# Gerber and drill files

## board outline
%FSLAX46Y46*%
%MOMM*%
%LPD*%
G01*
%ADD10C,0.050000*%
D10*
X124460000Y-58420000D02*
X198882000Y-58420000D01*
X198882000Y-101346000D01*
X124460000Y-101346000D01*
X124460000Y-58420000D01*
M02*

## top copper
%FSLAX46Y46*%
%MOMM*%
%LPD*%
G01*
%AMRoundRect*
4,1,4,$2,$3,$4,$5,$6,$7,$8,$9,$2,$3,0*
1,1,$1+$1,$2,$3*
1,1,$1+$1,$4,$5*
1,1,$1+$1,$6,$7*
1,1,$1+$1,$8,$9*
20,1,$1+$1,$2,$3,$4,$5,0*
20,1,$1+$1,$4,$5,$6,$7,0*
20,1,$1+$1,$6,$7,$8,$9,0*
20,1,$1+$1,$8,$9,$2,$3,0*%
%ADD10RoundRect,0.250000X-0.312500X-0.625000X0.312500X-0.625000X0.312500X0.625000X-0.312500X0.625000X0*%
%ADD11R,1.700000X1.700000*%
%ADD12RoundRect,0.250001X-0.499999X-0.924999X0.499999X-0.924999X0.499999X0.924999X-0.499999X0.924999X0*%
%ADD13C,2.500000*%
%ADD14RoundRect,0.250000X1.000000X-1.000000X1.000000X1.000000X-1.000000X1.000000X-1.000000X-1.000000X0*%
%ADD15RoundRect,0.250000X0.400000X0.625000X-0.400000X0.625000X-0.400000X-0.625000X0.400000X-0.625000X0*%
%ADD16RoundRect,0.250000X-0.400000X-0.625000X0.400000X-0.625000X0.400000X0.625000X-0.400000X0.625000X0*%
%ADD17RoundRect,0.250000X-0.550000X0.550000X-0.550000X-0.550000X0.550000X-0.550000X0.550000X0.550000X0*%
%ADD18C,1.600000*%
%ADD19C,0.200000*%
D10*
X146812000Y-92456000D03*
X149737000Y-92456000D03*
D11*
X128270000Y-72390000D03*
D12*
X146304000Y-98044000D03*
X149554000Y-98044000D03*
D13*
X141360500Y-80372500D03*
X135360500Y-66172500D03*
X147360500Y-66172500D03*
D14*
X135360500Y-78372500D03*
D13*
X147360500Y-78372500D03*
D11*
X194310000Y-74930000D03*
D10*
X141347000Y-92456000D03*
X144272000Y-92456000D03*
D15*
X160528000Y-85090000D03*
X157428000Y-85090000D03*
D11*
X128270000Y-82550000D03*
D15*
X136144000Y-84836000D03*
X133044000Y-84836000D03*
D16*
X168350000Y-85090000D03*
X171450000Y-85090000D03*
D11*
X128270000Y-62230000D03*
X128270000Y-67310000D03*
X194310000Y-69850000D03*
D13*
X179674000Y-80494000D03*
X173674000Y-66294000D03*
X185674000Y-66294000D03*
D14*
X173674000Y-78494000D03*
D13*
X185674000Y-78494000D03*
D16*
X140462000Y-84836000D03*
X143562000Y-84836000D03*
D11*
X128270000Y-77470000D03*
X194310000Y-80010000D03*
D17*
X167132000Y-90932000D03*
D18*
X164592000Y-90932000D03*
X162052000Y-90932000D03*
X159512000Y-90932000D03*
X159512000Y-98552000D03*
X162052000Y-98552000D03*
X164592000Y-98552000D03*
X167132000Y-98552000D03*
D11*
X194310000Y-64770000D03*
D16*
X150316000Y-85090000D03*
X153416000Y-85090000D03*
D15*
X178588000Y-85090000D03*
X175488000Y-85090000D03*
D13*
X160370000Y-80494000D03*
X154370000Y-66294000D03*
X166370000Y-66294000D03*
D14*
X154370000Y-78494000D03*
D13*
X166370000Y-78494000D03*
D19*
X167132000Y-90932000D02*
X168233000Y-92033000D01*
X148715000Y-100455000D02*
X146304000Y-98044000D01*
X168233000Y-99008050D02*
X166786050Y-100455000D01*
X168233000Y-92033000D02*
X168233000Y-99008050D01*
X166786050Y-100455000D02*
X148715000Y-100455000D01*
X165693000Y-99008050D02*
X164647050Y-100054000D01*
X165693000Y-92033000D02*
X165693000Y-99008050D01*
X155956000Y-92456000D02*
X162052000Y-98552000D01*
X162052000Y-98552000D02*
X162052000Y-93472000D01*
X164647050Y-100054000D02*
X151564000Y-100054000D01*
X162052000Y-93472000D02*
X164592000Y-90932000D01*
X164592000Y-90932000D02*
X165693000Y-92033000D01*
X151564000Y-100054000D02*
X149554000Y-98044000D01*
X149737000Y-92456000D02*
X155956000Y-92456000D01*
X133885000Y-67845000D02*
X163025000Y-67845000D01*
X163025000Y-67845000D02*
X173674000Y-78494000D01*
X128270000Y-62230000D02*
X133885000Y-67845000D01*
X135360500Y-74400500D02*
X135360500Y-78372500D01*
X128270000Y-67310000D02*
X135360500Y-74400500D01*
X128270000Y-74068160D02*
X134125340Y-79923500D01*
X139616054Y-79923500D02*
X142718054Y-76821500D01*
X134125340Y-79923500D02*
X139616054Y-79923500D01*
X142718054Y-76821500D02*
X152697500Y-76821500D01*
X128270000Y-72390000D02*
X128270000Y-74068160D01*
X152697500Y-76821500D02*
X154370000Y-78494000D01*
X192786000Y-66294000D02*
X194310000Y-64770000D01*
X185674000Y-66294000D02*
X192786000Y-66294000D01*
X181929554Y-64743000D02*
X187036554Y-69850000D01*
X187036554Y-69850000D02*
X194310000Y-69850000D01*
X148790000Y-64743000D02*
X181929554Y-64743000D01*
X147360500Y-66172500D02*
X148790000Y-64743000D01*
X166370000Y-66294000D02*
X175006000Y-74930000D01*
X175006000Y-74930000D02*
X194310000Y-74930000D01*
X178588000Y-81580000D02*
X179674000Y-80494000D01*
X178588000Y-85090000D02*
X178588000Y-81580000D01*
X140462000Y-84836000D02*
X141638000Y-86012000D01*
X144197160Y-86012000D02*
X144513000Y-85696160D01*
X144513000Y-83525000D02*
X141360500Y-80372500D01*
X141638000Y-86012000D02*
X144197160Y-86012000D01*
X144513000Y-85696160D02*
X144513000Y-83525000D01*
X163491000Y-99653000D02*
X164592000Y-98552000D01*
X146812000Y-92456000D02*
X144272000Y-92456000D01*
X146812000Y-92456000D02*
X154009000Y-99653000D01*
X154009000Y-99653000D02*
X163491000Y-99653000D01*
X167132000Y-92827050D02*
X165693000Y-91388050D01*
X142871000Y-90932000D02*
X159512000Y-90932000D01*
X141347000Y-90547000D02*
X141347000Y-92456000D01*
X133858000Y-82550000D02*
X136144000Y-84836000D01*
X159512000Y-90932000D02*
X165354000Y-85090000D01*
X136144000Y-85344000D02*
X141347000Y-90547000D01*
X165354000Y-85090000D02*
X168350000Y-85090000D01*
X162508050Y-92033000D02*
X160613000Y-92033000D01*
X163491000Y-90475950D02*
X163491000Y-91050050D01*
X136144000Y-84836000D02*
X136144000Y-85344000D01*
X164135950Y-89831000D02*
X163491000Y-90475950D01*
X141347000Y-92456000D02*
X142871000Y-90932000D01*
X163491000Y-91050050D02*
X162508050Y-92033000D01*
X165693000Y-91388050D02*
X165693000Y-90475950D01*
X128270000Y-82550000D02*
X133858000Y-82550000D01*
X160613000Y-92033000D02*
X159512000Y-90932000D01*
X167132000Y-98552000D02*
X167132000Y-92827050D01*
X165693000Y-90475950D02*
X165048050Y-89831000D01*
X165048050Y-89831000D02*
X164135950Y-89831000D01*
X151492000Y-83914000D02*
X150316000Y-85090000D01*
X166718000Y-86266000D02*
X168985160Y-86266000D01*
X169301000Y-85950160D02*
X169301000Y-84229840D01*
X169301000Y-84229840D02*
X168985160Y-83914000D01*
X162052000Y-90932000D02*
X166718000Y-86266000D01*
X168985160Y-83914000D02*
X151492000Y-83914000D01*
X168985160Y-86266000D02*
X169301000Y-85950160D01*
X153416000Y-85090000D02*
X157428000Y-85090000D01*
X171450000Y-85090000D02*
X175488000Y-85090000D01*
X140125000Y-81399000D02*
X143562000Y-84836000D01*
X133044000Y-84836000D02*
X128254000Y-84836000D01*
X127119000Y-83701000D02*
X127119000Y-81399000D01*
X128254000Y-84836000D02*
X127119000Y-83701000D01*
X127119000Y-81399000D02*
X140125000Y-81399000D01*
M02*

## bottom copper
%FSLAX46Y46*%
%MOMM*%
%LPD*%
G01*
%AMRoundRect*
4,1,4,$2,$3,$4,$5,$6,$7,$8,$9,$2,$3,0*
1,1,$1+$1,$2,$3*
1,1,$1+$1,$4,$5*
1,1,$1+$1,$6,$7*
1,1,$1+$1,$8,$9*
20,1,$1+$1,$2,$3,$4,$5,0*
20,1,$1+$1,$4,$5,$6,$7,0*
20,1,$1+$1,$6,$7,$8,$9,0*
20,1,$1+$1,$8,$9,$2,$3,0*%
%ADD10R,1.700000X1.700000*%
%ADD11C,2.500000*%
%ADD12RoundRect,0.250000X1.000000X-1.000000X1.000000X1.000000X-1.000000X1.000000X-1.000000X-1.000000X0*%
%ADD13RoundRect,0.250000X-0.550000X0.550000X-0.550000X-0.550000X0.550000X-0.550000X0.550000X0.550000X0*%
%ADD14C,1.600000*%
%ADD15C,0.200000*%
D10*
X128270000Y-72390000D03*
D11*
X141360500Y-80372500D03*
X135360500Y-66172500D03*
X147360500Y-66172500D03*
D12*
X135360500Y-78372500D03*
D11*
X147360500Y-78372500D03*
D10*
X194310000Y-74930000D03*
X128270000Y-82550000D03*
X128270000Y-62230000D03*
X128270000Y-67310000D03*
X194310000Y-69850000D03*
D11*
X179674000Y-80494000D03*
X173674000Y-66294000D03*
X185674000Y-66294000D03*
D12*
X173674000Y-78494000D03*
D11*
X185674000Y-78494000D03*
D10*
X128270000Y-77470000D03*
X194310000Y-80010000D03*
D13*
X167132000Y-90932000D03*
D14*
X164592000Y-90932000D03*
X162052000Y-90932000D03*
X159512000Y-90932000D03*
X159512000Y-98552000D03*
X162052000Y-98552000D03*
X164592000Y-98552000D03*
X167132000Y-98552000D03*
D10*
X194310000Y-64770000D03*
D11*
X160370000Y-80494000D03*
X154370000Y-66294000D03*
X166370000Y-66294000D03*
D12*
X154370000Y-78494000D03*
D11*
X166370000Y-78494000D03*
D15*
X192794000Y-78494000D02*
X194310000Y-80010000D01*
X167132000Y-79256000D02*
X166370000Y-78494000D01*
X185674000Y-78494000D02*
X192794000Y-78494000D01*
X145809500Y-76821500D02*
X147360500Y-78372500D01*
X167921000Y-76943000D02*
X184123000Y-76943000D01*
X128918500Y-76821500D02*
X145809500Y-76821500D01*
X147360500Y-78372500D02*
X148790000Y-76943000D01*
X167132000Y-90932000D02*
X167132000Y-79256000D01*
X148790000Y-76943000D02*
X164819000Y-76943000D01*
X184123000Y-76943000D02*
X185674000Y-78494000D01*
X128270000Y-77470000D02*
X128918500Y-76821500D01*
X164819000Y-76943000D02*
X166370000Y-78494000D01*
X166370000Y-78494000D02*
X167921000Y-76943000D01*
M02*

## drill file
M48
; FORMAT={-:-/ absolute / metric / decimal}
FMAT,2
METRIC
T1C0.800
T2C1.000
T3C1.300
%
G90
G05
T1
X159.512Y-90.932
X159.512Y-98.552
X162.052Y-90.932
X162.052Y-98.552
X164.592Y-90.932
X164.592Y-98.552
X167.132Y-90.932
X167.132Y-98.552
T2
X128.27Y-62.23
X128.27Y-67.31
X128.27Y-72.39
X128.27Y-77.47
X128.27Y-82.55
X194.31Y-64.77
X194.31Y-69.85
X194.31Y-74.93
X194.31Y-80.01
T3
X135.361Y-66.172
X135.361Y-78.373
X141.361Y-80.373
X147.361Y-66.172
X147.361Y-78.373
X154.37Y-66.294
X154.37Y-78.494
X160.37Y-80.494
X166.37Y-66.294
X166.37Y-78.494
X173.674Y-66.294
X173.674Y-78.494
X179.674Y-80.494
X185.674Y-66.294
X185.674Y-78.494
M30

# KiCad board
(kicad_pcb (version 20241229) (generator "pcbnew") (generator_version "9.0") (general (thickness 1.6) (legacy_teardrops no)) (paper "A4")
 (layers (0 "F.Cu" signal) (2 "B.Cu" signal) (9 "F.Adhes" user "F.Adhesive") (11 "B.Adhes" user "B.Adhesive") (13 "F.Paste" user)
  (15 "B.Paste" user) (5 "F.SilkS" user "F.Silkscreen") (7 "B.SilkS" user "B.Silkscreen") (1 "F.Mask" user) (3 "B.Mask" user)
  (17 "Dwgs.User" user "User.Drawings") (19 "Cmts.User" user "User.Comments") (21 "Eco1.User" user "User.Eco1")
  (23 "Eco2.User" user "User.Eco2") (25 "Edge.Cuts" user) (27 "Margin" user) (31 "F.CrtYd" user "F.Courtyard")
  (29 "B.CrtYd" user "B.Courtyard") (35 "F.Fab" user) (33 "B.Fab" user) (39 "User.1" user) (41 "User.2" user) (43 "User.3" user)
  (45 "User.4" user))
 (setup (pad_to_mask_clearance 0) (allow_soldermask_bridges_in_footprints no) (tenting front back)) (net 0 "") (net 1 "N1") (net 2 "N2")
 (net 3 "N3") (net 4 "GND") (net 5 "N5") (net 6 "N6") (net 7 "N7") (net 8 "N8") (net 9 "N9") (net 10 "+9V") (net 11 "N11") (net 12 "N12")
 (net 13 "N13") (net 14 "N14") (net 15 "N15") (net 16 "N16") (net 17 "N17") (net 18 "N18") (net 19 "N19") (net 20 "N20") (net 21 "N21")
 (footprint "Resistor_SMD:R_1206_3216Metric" (layer "F.Cu") (at 148.2745 92.456)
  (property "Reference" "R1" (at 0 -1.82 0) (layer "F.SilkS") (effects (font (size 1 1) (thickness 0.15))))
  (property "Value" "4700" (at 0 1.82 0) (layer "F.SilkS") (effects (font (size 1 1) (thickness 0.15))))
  (pad "1" smd roundrect (at -1.4625 0) (size 1.125 1.75) (layers "F.Cu" "F.Mask" "F.Paste") (roundrect_rratio 0.222222) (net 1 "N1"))
  (pad "2" smd roundrect (at 1.4625 0) (size 1.125 1.75) (layers "F.Cu" "F.Mask" "F.Paste") (roundrect_rratio 0.222222) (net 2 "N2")))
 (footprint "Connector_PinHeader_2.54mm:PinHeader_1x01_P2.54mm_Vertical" (layer "F.Cu") (at 128.27 72.39 -90)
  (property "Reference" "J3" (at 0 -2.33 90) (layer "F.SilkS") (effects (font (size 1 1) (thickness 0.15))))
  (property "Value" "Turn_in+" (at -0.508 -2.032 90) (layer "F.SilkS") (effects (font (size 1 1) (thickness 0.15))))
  (pad "1" thru_hole rect (at 0 0 270) (size 1.7 1.7) (drill 1) (layers "*.Cu" "*.Mask") (remove_unused_layers no) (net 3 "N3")))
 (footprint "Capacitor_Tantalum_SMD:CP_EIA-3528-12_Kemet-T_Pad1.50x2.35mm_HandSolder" (layer "F.Cu") (at 147.929 98.044)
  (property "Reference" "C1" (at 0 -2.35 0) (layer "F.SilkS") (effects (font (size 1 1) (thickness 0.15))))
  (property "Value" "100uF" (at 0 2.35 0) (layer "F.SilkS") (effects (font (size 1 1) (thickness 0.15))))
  (pad "1" smd roundrect (at -1.625 0) (size 1.5 2.35) (layers "F.Cu" "F.Mask" "F.Paste") (roundrect_rratio 0.166667) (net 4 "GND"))
  (pad "2" smd roundrect (at 1.625 0) (size 1.5 2.35) (layers "F.Cu" "F.Mask" "F.Paste") (roundrect_rratio 0.166667) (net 2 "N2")))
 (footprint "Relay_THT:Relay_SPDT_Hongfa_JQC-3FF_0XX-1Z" (layer "F.Cu") (at 135.3605 78.3725 90)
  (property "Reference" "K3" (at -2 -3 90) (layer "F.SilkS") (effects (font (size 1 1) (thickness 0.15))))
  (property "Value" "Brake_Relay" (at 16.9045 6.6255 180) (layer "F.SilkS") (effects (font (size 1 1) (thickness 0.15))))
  (pad "11" thru_hole circle (at -2 6 90) (size 2.5 2.5) (drill 1.3) (layers "*.Cu" "*.Mask") (remove_unused_layers no) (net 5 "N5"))
  (pad "12" thru_hole circle (at 12.2 0 90) (size 2.5 2.5) (drill 1.3) (layers "*.Cu" "*.Mask") (remove_unused_layers no) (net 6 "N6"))
  (pad "14" thru_hole circle (at 12.2 12 90) (size 2.5 2.5) (drill 1.3) (layers "*.Cu" "*.Mask") (remove_unused_layers no) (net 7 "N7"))
  (pad "A1" thru_hole roundrect (at 0 0 90) (size 2.5 2.5) (drill 1.3) (layers "*.Cu" "*.Mask") (remove_unused_layers no)
   (roundrect_rratio 0.1) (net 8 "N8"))
  (pad "A2" thru_hole circle (at 0 12 90) (size 2.5 2.5) (drill 1.3) (layers "*.Cu" "*.Mask") (remove_unused_layers no) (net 4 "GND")))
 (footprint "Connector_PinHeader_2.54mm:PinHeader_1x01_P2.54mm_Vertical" (layer "F.Cu") (at 194.31 74.93 -90)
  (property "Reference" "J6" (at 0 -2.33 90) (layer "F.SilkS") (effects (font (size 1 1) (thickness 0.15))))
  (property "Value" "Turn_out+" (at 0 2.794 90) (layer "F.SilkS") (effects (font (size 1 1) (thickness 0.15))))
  (pad "1" thru_hole rect (at 0 0 270) (size 1.7 1.7) (drill 1) (layers "*.Cu" "*.Mask") (remove_unused_layers no) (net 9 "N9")))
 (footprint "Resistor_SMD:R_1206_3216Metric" (layer "F.Cu") (at 142.8095 92.456)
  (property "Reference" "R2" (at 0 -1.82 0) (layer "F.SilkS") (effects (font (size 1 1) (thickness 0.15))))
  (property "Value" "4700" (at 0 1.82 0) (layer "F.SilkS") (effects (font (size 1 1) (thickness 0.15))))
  (pad "1" smd roundrect (at -1.4625 0) (size 1.125 1.75) (layers "F.Cu" "F.Mask" "F.Paste") (roundrect_rratio 0.222222) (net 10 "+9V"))
  (pad "2" smd roundrect (at 1.4625 0) (size 1.125 1.75) (layers "F.Cu" "F.Mask" "F.Paste") (roundrect_rratio 0.222222) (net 1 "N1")))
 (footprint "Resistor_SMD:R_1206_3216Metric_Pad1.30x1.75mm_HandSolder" (layer "F.Cu") (at 158.978 85.09 180)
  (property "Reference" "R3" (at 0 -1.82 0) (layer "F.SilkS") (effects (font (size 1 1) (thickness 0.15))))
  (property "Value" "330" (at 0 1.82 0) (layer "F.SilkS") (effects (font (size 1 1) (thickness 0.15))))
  (pad "1" smd roundrect (at -1.55 0 180) (size 1.3 1.75) (layers "F.Cu" "F.Mask" "F.Paste") (roundrect_rratio 0.192308) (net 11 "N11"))
  (pad "2" smd roundrect (at 1.55 0 180) (size 1.3 1.75) (layers "F.Cu" "F.Mask" "F.Paste") (roundrect_rratio 0.192308) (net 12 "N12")))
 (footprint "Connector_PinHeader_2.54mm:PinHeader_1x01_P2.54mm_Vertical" (layer "F.Cu") (at 128.27 82.55 -90)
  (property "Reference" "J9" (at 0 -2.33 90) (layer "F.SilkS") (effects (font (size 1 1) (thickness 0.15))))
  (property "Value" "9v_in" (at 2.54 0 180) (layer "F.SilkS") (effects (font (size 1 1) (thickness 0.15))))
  (pad "1" thru_hole rect (at 0 0 270) (size 1.7 1.7) (drill 1) (layers "*.Cu" "*.Mask") (remove_unused_layers no) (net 10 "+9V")))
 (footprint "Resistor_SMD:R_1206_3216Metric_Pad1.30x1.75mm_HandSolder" (layer "F.Cu") (at 134.594 84.836 180)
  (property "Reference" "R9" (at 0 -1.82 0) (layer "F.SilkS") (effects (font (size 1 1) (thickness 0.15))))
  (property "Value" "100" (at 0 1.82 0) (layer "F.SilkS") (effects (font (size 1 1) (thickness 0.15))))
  (pad "1" smd roundrect (at -1.55 0 180) (size 1.3 1.75) (layers "F.Cu" "F.Mask" "F.Paste") (roundrect_rratio 0.192308) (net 10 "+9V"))
  (pad "2" smd roundrect (at 1.55 0 180) (size 1.3 1.75) (layers "F.Cu" "F.Mask" "F.Paste") (roundrect_rratio 0.192308) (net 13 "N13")))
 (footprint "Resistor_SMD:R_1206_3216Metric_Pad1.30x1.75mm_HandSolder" (layer "F.Cu") (at 169.9 85.09)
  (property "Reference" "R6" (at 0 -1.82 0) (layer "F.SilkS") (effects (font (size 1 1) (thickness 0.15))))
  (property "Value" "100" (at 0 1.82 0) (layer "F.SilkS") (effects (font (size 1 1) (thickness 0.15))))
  (pad "1" smd roundrect (at -1.55 0) (size 1.3 1.75) (layers "F.Cu" "F.Mask" "F.Paste") (roundrect_rratio 0.192308) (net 10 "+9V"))
  (pad "2" smd roundrect (at 1.55 0) (size 1.3 1.75) (layers "F.Cu" "F.Mask" "F.Paste") (roundrect_rratio 0.192308) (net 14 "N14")))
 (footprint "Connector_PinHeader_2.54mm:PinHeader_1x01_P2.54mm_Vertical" (layer "F.Cu") (at 128.27 62.23 -90)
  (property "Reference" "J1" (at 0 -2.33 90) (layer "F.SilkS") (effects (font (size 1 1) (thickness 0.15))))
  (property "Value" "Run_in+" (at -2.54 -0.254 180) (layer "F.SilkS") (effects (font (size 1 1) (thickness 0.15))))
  (pad "1" thru_hole rect (at 0 0 270) (size 1.7 1.7) (drill 1) (layers "*.Cu" "*.Mask") (remove_unused_layers no) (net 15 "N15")))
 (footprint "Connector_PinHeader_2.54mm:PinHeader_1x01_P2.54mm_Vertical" (layer "F.Cu") (at 128.27 67.31 -90)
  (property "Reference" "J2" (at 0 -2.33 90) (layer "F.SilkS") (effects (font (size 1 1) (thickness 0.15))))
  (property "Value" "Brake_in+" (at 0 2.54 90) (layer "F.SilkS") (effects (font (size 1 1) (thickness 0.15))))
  (pad "1" thru_hole rect (at 0 0 270) (size 1.7 1.7) (drill 1) (layers "*.Cu" "*.Mask") (remove_unused_layers no) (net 8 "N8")))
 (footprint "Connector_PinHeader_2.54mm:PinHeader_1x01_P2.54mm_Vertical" (layer "F.Cu") (at 194.31 69.85 -90)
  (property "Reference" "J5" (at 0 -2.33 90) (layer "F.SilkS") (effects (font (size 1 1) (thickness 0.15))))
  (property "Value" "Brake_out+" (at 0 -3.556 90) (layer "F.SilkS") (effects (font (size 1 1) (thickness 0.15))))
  (pad "1" thru_hole rect (at 0 0 270) (size 1.7 1.7) (drill 1) (layers "*.Cu" "*.Mask") (remove_unused_layers no) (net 7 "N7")))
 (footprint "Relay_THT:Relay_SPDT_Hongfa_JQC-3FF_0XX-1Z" (layer "F.Cu") (at 173.674 78.494 90)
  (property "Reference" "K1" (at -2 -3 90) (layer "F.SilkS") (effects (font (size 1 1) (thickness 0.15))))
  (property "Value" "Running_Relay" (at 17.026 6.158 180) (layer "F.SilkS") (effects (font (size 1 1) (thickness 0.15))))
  (pad "11" thru_hole circle (at -2 6 90) (size 2.5 2.5) (drill 1.3) (layers "*.Cu" "*.Mask") (remove_unused_layers no) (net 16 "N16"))
  (pad "12" thru_hole circle (at 12.2 0 90) (size 2.5 2.5) (drill 1.3) (layers "*.Cu" "*.Mask") (remove_unused_layers no) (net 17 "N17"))
  (pad "14" thru_hole circle (at 12.2 12 90) (size 2.5 2.5) (drill 1.3) (layers "*.Cu" "*.Mask") (remove_unused_layers no) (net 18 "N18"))
  (pad "A1" thru_hole roundrect (at 0 0 90) (size 2.5 2.5) (drill 1.3) (layers "*.Cu" "*.Mask") (remove_unused_layers no)
   (roundrect_rratio 0.1) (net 15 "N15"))
  (pad "A2" thru_hole circle (at 0 12 90) (size 2.5 2.5) (drill 1.3) (layers "*.Cu" "*.Mask") (remove_unused_layers no) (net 4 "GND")))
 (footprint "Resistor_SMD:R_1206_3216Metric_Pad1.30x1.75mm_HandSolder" (layer "F.Cu") (at 142.012 84.836)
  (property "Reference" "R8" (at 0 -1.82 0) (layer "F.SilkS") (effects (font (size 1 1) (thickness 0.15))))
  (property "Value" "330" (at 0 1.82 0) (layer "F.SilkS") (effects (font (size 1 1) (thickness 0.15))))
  (pad "1" smd roundrect (at -1.55 0) (size 1.3 1.75) (layers "F.Cu" "F.Mask" "F.Paste") (roundrect_rratio 0.192308) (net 5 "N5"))
  (pad "2" smd roundrect (at 1.55 0) (size 1.3 1.75) (layers "F.Cu" "F.Mask" "F.Paste") (roundrect_rratio 0.192308) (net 13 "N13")))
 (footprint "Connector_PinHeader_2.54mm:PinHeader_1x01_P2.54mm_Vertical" (layer "F.Cu") (at 128.27 77.47 -90)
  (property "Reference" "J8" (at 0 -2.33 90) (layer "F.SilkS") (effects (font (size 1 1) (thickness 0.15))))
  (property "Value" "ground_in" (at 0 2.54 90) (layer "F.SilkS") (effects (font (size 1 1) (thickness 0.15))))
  (pad "1" thru_hole rect (at 0 0 270) (size 1.7 1.7) (drill 1) (layers "*.Cu" "*.Mask") (remove_unused_layers no) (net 4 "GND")))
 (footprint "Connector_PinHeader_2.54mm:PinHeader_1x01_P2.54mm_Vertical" (layer "F.Cu") (at 194.31 80.01 -90)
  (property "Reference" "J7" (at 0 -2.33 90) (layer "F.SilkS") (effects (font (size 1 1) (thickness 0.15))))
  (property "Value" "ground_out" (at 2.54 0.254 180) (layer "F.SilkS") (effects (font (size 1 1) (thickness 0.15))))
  (pad "1" thru_hole rect (at 0 0 270) (size 1.7 1.7) (drill 1) (layers "*.Cu" "*.Mask") (remove_unused_layers no) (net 4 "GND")))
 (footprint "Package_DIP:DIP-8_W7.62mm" (layer "F.Cu") (at 167.132 90.932 -90)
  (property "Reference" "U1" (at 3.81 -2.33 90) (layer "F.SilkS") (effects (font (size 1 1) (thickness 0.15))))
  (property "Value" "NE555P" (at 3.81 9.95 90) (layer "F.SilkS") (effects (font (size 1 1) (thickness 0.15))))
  (pad "1" thru_hole roundrect (at 0 0 270) (size 1.6 1.6) (drill 0.8) (layers "*.Cu" "*.Mask") (remove_unused_layers no)
   (roundrect_rratio 0.15625) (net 4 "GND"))
  (pad "2" thru_hole circle (at 0 2.54 270) (size 1.6 1.6) (drill 0.8) (layers "*.Cu" "*.Mask") (remove_unused_layers no) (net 2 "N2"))
  (pad "3" thru_hole circle (at 0 5.08 270) (size 1.6 1.6) (drill 0.8) (layers "*.Cu" "*.Mask") (remove_unused_layers no) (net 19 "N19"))
  (pad "4" thru_hole circle (at 0 7.62 270) (size 1.6 1.6) (drill 0.8) (layers "*.Cu" "*.Mask") (remove_unused_layers no) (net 10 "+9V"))
  (pad "5" thru_hole circle (at 7.62 7.62 270) (size 1.6 1.6) (drill 0.8) (layers "*.Cu" "*.Mask") (remove_unused_layers no) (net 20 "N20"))
  (pad "6" thru_hole circle (at 7.62 5.08 270) (size 1.6 1.6) (drill 0.8) (layers "*.Cu" "*.Mask") (remove_unused_layers no) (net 2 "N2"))
  (pad "7" thru_hole circle (at 7.62 2.54 270) (size 1.6 1.6) (drill 0.8) (layers "*.Cu" "*.Mask") (remove_unused_layers no) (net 1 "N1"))
  (pad "8" thru_hole circle (at 7.62 0 270) (size 1.6 1.6) (drill 0.8) (layers "*.Cu" "*.Mask") (remove_unused_layers no) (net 10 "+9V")))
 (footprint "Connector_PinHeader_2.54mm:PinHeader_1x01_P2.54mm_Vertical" (layer "F.Cu") (at 194.31 64.77 -90)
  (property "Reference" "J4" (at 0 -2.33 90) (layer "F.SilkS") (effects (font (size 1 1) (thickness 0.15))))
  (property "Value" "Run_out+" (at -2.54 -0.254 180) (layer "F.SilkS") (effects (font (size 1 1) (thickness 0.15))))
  (pad "1" thru_hole rect (at 0 0 270) (size 1.7 1.7) (drill 1) (layers "*.Cu" "*.Mask") (remove_unused_layers no) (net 18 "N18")))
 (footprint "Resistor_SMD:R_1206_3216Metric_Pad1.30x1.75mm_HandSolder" (layer "F.Cu") (at 151.866 85.09)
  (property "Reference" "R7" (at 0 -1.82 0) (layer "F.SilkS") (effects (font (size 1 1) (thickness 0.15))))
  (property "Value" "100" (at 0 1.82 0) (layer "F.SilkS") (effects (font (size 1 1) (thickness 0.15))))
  (pad "1" smd roundrect (at -1.55 0) (size 1.3 1.75) (layers "F.Cu" "F.Mask" "F.Paste") (roundrect_rratio 0.192308) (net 19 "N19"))
  (pad "2" smd roundrect (at 1.55 0) (size 1.3 1.75) (layers "F.Cu" "F.Mask" "F.Paste") (roundrect_rratio 0.192308) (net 12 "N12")))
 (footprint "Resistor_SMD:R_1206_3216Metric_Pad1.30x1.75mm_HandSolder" (layer "F.Cu") (at 177.038 85.09 180)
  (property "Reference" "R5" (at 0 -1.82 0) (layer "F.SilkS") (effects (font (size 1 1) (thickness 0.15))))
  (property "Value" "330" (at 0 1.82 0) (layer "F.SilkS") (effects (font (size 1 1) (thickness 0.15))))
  (pad "1" smd roundrect (at -1.55 0 180) (size 1.3 1.75) (layers "F.Cu" "F.Mask" "F.Paste") (roundrect_rratio 0.192308) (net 16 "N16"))
  (pad "2" smd roundrect (at 1.55 0 180) (size 1.3 1.75) (layers "F.Cu" "F.Mask" "F.Paste") (roundrect_rratio 0.192308) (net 14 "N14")))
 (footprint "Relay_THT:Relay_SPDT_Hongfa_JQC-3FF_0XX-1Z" (layer "F.Cu") (at 154.37 78.494 90)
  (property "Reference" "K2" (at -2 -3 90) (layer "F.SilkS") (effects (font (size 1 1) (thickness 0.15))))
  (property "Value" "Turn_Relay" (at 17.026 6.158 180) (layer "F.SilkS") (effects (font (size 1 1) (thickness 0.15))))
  (pad "11" thru_hole circle (at -2 6 90) (size 2.5 2.5) (drill 1.3) (layers "*.Cu" "*.Mask") (remove_unused_layers no) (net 11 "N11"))
  (pad "12" thru_hole circle (at 12.2 0 90) (size 2.5 2.5) (drill 1.3) (layers "*.Cu" "*.Mask") (remove_unused_layers no) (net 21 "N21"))
  (pad "14" thru_hole circle (at 12.2 12 90) (size 2.5 2.5) (drill 1.3) (layers "*.Cu" "*.Mask") (remove_unused_layers no) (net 9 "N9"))
  (pad "A1" thru_hole roundrect (at 0 0 90) (size 2.5 2.5) (drill 1.3) (layers "*.Cu" "*.Mask") (remove_unused_layers no)
   (roundrect_rratio 0.1) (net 3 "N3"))
  (pad "A2" thru_hole circle (at 0 12 90) (size 2.5 2.5) (drill 1.3) (layers "*.Cu" "*.Mask") (remove_unused_layers no) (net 4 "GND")))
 (gr_rect (start 124.46 58.42) (end 198.882 101.346) (stroke (width 0.05) (type default)) (fill no) (layer "Edge.Cuts"))
 (segment (start 167.132 90.932) (end 168.233 92.033) (width 0.2) (layer "F.Cu") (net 4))
 (segment (start 148.715 100.455) (end 146.304 98.044) (width 0.2) (layer "F.Cu") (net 4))
 (segment (start 168.233 99.00805) (end 166.78605 100.455) (width 0.2) (layer "F.Cu") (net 4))
 (segment (start 168.233 92.033) (end 168.233 99.00805) (width 0.2) (layer "F.Cu") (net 4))
 (segment (start 166.78605 100.455) (end 148.715 100.455) (width 0.2) (layer "F.Cu") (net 4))
 (segment (start 192.794 78.494) (end 194.31 80.01) (width 0.2) (layer "B.Cu") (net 4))
 (segment (start 167.132 79.256) (end 166.37 78.494) (width 0.2) (layer "B.Cu") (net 4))
 (segment (start 185.674 78.494) (end 192.794 78.494) (width 0.2) (layer "B.Cu") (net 4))
 (segment (start 145.8095 76.8215) (end 147.3605 78.3725) (width 0.2) (layer "B.Cu") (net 4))
 (segment (start 167.921 76.943) (end 184.123 76.943) (width 0.2) (layer "B.Cu") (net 4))
 (segment (start 128.9185 76.8215) (end 145.8095 76.8215) (width 0.2) (layer "B.Cu") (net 4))
 (segment (start 147.3605 78.3725) (end 148.79 76.943) (width 0.2) (layer "B.Cu") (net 4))
 (segment (start 167.132 90.932) (end 167.132 79.256) (width 0.2) (layer "B.Cu") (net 4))
 (segment (start 148.79 76.943) (end 164.819 76.943) (width 0.2) (layer "B.Cu") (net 4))
 (segment (start 184.123 76.943) (end 185.674 78.494) (width 0.2) (layer "B.Cu") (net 4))
 (segment (start 128.27 77.47) (end 128.9185 76.8215) (width 0.2) (layer "B.Cu") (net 4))
 (segment (start 164.819 76.943) (end 166.37 78.494) (width 0.2) (layer "B.Cu") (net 4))
 (segment (start 166.37 78.494) (end 167.921 76.943) (width 0.2) (layer "B.Cu") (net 4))
 (segment (start 165.693 99.00805) (end 164.64705 100.054) (width 0.2) (layer "F.Cu") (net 2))
 (segment (start 165.693 92.033) (end 165.693 99.00805) (width 0.2) (layer "F.Cu") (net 2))
 (segment (start 155.956 92.456) (end 162.052 98.552) (width 0.2) (layer "F.Cu") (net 2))
 (segment (start 162.052 98.552) (end 162.052 93.472) (width 0.2) (layer "F.Cu") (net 2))
 (segment (start 164.64705 100.054) (end 151.564 100.054) (width 0.2) (layer "F.Cu") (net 2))
 (segment (start 162.052 93.472) (end 164.592 90.932) (width 0.2) (layer "F.Cu") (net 2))
 (segment (start 164.592 90.932) (end 165.693 92.033) (width 0.2) (layer "F.Cu") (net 2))
 (segment (start 151.564 100.054) (end 149.554 98.044) (width 0.2) (layer "F.Cu") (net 2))
 (segment (start 149.737 92.456) (end 155.956 92.456) (width 0.2) (layer "F.Cu") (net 2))
 (segment (start 133.885 67.845) (end 163.025 67.845) (width 0.2) (layer "F.Cu") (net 15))
 (segment (start 163.025 67.845) (end 173.674 78.494) (width 0.2) (layer "F.Cu") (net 15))
 (segment (start 128.27 62.23) (end 133.885 67.845) (width 0.2) (layer "F.Cu") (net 15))
 (segment (start 135.3605 74.4005) (end 135.3605 78.3725) (width 0.2) (layer "F.Cu") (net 8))
 (segment (start 128.27 67.31) (end 135.3605 74.4005) (width 0.2) (layer "F.Cu") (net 8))
 (segment (start 128.27 74.06816) (end 134.12534 79.9235) (width 0.2) (layer "F.Cu") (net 3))
 (segment (start 139.616054 79.9235) (end 142.718054 76.8215) (width 0.2) (layer "F.Cu") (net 3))
 (segment (start 134.12534 79.9235) (end 139.616054 79.9235) (width 0.2) (layer "F.Cu") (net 3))
 (segment (start 142.718054 76.8215) (end 152.6975 76.8215) (width 0.2) (layer "F.Cu") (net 3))
 (segment (start 128.27 72.39) (end 128.27 74.06816) (width 0.2) (layer "F.Cu") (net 3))
 (segment (start 152.6975 76.8215) (end 154.37 78.494) (width 0.2) (layer "F.Cu") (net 3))
 (segment (start 192.786 66.294) (end 194.31 64.77) (width 0.2) (layer "F.Cu") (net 18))
 (segment (start 185.674 66.294) (end 192.786 66.294) (width 0.2) (layer "F.Cu") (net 18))
 (segment (start 181.929554 64.743) (end 187.036554 69.85) (width 0.2) (layer "F.Cu") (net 7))
 (segment (start 187.036554 69.85) (end 194.31 69.85) (width 0.2) (layer "F.Cu") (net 7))
 (segment (start 148.79 64.743) (end 181.929554 64.743) (width 0.2) (layer "F.Cu") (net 7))
 (segment (start 147.3605 66.1725) (end 148.79 64.743) (width 0.2) (layer "F.Cu") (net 7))
 (segment (start 166.37 66.294) (end 175.006 74.93) (width 0.2) (layer "F.Cu") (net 9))
 (segment (start 175.006 74.93) (end 194.31 74.93) (width 0.2) (layer "F.Cu") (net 9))
 (segment (start 178.588 81.58) (end 179.674 80.494) (width 0.2) (layer "F.Cu") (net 16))
 (segment (start 178.588 85.09) (end 178.588 81.58) (width 0.2) (layer "F.Cu") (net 16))
 (segment (start 140.462 84.836) (end 141.638 86.012) (width 0.2) (layer "F.Cu") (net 5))
 (segment (start 144.19716 86.012) (end 144.513 85.69616) (width 0.2) (layer "F.Cu") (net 5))
 (segment (start 144.513 83.525) (end 141.3605 80.3725) (width 0.2) (layer "F.Cu") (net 5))
 (segment (start 141.638 86.012) (end 144.19716 86.012) (width 0.2) (layer "F.Cu") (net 5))
 (segment (start 144.513 85.69616) (end 144.513 83.525) (width 0.2) (layer "F.Cu") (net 5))
 (segment (start 163.491 99.653) (end 164.592 98.552) (width 0.2) (layer "F.Cu") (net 1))
 (segment (start 146.812 92.456) (end 144.272 92.456) (width 0.2) (layer "F.Cu") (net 1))
 (segment (start 146.812 92.456) (end 154.009 99.653) (width 0.2) (layer "F.Cu") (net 1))
 (segment (start 154.009 99.653) (end 163.491 99.653) (width 0.2) (layer "F.Cu") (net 1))
 (segment (start 167.132 92.82705) (end 165.693 91.38805) (width 0.2) (layer "F.Cu") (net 10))
 (segment (start 142.871 90.932) (end 159.512 90.932) (width 0.2) (layer "F.Cu") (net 10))
 (segment (start 141.347 90.547) (end 141.347 92.456) (width 0.2) (layer "F.Cu") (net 10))
 (segment (start 133.858 82.55) (end 136.144 84.836) (width 0.2) (layer "F.Cu") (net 10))
 (segment (start 159.512 90.932) (end 165.354 85.09) (width 0.2) (layer "F.Cu") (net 10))
 (segment (start 136.144 85.344) (end 141.347 90.547) (width 0.2) (layer "F.Cu") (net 10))
 (segment (start 165.354 85.09) (end 168.35 85.09) (width 0.2) (layer "F.Cu") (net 10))
 (segment (start 162.50805 92.033) (end 160.613 92.033) (width 0.2) (layer "F.Cu") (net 10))
 (segment (start 163.491 90.47595) (end 163.491 91.05005) (width 0.2) (layer "F.Cu") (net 10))
 (segment (start 136.144 84.836) (end 136.144 85.344) (width 0.2) (layer "F.Cu") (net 10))
 (segment (start 164.13595 89.831) (end 163.491 90.47595) (width 0.2) (layer "F.Cu") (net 10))
 (segment (start 141.347 92.456) (end 142.871 90.932) (width 0.2) (layer "F.Cu") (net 10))
 (segment (start 163.491 91.05005) (end 162.50805 92.033) (width 0.2) (layer "F.Cu") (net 10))
 (segment (start 165.693 91.38805) (end 165.693 90.47595) (width 0.2) (layer "F.Cu") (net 10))
 (segment (start 128.27 82.55) (end 133.858 82.55) (width 0.2) (layer "F.Cu") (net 10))
 (segment (start 160.613 92.033) (end 159.512 90.932) (width 0.2) (layer "F.Cu") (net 10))
 (segment (start 167.132 98.552) (end 167.132 92.82705) (width 0.2) (layer "F.Cu") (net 10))
 (segment (start 165.693 90.47595) (end 165.04805 89.831) (width 0.2) (layer "F.Cu") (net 10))
 (segment (start 165.04805 89.831) (end 164.13595 89.831) (width 0.2) (layer "F.Cu") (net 10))
 (segment (start 151.492 83.914) (end 150.316 85.09) (width 0.2) (layer "F.Cu") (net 19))
 (segment (start 166.718 86.266) (end 168.98516 86.266) (width 0.2) (layer "F.Cu") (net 19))
 (segment (start 169.301 85.95016) (end 169.301 84.22984) (width 0.2) (layer "F.Cu") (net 19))
 (segment (start 169.301 84.22984) (end 168.98516 83.914) (width 0.2) (layer "F.Cu") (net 19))
 (segment (start 162.052 90.932) (end 166.718 86.266) (width 0.2) (layer "F.Cu") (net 19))
 (segment (start 168.98516 83.914) (end 151.492 83.914) (width 0.2) (layer "F.Cu") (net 19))
 (segment (start 168.98516 86.266) (end 169.301 85.95016) (width 0.2) (layer "F.Cu") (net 19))
 (segment (start 153.416 85.09) (end 157.428 85.09) (width 0.2) (layer "F.Cu") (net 12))
 (segment (start 171.45 85.09) (end 175.488 85.09) (width 0.2) (layer "F.Cu") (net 14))
 (segment (start 140.125 81.399) (end 143.562 84.836) (width 0.2) (layer "F.Cu") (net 13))
 (segment (start 133.044 84.836) (end 128.254 84.836) (width 0.2) (layer "F.Cu") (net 13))
 (segment (start 127.119 83.701) (end 127.119 81.399) (width 0.2) (layer "F.Cu") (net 13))
 (segment (start 128.254 84.836) (end 127.119 83.701) (width 0.2) (layer "F.Cu") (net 13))
 (segment (start 127.119 81.399) (end 140.125 81.399) (width 0.2) (layer "F.Cu") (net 13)))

